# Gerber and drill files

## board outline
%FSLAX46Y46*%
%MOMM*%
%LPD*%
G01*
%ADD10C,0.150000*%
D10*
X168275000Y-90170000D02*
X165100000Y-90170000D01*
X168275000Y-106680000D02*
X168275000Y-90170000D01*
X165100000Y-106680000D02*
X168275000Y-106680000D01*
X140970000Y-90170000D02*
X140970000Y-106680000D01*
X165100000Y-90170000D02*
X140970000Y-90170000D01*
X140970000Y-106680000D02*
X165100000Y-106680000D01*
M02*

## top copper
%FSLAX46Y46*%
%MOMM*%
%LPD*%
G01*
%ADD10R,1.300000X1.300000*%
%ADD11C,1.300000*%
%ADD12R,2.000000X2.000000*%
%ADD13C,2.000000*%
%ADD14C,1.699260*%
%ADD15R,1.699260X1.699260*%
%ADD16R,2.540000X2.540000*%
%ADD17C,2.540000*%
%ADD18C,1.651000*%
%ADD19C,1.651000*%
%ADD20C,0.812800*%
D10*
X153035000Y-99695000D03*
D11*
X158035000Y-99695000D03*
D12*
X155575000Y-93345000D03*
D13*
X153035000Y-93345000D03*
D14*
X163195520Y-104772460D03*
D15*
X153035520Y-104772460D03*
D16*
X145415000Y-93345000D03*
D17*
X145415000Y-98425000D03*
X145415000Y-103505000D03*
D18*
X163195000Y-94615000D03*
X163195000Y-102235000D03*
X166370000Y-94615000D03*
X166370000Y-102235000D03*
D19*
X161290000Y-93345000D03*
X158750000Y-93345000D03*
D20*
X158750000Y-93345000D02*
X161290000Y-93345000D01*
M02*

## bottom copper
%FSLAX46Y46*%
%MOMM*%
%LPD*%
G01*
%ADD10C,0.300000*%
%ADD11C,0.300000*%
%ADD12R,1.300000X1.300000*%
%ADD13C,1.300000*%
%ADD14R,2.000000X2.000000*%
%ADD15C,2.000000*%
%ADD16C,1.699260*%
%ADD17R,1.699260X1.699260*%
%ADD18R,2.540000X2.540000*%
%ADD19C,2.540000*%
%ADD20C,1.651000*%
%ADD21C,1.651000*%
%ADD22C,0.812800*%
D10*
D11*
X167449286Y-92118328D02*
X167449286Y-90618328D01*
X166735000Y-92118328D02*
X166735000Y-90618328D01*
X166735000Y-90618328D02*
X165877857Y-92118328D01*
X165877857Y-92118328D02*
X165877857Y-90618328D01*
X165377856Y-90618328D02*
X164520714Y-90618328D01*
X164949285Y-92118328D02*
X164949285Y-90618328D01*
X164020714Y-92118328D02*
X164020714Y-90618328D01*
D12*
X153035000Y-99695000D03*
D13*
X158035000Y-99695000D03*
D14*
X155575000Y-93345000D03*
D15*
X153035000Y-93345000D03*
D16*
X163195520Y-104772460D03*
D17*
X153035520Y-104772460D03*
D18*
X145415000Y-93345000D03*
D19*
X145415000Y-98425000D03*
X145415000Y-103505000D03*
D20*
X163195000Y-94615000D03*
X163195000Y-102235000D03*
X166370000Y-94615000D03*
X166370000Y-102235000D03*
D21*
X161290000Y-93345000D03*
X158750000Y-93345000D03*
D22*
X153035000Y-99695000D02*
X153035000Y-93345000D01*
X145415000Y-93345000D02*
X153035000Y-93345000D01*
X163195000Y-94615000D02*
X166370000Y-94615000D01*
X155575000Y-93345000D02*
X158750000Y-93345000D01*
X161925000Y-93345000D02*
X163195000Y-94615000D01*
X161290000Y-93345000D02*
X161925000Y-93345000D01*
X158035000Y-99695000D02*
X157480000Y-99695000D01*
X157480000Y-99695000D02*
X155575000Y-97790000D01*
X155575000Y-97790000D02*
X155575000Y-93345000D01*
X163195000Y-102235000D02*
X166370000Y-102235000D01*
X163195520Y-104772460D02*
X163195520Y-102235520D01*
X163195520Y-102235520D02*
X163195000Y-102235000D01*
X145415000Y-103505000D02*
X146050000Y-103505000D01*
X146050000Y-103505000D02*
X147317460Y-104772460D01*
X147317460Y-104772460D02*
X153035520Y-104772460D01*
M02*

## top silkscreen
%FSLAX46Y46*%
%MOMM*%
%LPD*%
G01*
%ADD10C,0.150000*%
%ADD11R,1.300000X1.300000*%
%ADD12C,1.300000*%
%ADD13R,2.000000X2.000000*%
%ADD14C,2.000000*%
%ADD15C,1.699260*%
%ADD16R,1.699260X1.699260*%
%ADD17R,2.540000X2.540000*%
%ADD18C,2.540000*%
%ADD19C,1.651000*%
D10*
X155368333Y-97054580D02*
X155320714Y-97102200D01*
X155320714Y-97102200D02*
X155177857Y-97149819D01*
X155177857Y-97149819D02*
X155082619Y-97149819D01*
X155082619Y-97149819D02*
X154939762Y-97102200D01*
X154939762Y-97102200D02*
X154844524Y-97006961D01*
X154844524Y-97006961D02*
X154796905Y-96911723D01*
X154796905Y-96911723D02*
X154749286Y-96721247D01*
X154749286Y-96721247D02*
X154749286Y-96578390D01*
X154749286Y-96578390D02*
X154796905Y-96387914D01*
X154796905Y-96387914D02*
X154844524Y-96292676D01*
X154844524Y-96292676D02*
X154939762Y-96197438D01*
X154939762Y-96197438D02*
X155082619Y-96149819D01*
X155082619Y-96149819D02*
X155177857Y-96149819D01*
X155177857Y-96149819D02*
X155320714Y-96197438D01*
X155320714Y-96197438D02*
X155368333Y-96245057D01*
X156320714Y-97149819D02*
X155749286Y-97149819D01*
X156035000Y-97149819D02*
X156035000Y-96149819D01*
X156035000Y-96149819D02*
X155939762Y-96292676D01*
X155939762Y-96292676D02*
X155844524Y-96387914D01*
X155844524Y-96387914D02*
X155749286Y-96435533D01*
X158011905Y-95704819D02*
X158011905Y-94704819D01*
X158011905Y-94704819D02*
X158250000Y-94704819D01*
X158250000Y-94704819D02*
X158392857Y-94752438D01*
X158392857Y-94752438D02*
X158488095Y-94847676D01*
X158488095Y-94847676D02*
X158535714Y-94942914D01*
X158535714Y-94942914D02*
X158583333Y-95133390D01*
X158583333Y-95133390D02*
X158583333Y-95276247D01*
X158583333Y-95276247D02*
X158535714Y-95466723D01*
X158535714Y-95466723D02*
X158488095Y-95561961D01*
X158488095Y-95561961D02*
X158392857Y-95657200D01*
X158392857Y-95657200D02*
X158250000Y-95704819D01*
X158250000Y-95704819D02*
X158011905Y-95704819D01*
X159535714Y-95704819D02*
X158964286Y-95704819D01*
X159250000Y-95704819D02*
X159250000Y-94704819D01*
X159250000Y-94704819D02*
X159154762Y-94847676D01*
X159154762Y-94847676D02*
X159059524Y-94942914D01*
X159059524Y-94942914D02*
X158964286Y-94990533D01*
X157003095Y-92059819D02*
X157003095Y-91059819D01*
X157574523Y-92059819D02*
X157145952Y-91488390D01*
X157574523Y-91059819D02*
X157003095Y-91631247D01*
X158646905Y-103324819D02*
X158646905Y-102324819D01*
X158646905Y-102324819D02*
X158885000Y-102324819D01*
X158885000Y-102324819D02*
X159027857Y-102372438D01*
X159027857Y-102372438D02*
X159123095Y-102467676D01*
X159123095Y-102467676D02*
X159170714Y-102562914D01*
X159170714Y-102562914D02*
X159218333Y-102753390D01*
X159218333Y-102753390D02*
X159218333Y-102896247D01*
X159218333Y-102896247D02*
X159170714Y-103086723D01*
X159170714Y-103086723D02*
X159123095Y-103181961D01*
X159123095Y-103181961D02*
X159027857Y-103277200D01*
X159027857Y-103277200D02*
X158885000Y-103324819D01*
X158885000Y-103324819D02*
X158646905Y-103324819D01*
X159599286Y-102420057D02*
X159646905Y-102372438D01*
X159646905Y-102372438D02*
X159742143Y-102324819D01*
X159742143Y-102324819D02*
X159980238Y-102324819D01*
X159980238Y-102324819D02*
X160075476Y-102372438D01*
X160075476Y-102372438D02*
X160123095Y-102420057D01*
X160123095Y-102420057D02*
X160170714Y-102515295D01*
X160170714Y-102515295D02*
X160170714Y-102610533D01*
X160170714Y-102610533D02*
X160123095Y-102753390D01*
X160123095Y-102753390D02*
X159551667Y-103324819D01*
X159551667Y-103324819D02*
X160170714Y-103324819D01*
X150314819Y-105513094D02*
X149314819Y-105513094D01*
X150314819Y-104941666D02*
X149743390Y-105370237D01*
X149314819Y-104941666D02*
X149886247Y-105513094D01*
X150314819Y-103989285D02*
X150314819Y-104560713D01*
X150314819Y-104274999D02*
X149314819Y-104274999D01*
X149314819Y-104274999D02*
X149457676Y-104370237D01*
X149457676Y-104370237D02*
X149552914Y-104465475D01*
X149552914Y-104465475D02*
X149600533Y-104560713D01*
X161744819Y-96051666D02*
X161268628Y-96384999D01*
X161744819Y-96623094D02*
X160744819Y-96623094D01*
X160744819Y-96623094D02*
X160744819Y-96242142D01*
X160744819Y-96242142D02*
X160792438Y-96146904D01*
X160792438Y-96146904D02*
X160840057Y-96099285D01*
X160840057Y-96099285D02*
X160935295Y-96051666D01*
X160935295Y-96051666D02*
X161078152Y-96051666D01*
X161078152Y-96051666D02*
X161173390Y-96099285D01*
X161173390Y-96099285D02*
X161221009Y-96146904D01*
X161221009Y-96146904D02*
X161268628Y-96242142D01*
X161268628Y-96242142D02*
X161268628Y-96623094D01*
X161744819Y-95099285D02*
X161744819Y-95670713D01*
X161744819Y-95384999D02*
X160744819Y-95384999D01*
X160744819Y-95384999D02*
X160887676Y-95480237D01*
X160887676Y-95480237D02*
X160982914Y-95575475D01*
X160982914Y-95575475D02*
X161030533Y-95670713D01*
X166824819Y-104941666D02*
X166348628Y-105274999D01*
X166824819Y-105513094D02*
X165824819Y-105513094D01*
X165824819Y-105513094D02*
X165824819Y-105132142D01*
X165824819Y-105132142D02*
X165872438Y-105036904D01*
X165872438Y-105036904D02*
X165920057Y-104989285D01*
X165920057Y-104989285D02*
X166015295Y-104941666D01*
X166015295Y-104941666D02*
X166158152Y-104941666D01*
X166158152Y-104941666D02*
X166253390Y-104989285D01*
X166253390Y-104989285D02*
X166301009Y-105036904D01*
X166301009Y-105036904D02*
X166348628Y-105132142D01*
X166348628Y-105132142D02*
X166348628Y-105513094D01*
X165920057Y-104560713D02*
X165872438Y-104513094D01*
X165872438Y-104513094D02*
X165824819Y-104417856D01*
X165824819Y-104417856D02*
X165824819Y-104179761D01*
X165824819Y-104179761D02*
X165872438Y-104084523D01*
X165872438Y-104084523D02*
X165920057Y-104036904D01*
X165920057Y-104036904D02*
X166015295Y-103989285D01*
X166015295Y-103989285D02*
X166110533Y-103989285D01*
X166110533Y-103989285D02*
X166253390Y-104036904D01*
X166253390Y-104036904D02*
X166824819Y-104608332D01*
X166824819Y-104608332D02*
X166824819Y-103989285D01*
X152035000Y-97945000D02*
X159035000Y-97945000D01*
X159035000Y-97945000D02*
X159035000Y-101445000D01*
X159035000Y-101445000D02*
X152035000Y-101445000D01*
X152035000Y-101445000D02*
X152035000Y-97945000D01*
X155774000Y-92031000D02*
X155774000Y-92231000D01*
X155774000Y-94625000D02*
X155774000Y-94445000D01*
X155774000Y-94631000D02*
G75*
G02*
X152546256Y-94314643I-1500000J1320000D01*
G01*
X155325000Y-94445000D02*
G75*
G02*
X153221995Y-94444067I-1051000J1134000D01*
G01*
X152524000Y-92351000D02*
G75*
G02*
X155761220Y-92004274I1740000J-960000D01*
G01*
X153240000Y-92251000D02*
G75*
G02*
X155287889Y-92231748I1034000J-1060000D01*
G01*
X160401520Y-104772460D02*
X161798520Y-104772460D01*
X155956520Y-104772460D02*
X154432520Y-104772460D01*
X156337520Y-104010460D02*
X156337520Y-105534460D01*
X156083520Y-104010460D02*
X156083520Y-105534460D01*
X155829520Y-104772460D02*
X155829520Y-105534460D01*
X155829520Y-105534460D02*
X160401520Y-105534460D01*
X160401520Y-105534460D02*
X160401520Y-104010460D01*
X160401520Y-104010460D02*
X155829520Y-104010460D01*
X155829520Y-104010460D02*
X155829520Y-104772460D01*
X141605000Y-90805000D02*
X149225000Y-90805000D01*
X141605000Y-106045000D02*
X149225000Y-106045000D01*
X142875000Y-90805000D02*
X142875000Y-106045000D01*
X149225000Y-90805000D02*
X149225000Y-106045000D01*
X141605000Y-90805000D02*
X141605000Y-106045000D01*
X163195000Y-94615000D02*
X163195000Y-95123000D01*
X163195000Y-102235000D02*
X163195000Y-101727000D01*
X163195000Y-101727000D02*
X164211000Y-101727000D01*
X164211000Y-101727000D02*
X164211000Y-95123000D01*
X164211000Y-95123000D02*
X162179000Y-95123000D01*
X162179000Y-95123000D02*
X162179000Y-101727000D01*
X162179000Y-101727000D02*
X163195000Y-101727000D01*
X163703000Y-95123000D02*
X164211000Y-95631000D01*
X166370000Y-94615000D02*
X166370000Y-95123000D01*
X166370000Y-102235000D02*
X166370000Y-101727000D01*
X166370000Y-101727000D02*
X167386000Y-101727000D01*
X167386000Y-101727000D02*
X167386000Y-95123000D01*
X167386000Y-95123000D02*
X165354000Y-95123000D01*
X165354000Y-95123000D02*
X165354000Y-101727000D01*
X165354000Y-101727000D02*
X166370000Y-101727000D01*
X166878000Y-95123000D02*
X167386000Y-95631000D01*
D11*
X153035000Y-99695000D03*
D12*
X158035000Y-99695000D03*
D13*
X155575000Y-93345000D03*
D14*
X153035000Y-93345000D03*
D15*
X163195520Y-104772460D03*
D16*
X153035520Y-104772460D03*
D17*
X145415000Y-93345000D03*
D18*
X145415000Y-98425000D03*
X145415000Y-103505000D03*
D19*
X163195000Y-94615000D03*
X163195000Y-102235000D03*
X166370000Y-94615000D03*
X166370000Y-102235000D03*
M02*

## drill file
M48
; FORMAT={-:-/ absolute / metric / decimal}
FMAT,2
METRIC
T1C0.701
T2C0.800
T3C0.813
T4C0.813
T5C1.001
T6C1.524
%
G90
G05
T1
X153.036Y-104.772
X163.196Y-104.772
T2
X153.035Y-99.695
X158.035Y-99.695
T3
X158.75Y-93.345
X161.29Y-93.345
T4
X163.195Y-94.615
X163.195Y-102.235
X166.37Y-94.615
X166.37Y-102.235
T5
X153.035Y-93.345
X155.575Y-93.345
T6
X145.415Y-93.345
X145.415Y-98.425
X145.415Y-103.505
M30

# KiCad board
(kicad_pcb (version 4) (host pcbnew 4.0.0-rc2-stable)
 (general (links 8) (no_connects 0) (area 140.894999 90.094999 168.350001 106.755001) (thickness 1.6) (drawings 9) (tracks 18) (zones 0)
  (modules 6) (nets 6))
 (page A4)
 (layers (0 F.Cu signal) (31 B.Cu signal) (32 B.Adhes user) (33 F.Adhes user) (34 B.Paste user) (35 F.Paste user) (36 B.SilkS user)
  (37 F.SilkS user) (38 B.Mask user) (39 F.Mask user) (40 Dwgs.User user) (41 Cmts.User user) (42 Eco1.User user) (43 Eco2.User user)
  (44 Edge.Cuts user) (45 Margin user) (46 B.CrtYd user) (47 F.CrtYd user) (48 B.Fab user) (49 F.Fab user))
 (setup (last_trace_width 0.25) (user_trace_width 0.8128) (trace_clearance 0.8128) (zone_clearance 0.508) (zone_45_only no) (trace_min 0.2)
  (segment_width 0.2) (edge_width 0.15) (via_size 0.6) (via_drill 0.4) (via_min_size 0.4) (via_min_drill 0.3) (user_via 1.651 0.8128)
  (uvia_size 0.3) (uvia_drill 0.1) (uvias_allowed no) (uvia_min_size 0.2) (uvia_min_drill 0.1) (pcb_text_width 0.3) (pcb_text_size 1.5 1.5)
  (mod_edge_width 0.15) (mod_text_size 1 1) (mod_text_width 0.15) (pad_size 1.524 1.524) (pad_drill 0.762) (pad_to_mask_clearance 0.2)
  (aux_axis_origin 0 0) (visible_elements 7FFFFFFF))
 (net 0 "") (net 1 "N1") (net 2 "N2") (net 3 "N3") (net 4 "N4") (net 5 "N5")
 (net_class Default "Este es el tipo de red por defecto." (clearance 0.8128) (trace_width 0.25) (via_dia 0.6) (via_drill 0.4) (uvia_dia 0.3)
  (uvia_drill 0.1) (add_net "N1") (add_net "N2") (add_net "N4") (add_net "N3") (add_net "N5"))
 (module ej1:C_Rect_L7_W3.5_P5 (layer F.Cu) (at 153.035 99.695)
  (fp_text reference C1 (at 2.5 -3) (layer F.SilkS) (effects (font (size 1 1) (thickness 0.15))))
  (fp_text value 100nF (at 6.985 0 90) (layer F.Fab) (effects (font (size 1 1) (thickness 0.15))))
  (fp_line (start -1 -1.75) (end 6 -1.75) (layer F.SilkS) (width 0.15))
  (fp_line (start 6 -1.75) (end 6 1.75) (layer F.SilkS) (width 0.15))
  (fp_line (start 6 1.75) (end -1 1.75) (layer F.SilkS) (width 0.15))
  (fp_line (start -1 1.75) (end -1 -1.75) (layer F.SilkS) (width 0.15))
  (pad 1 thru_hole rect (at 0 0) (size 1.3 1.3) (drill 0.8) (layers *.Cu *.Mask F.SilkS) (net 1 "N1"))
  (pad 2 thru_hole circle (at 5 0) (size 1.3 1.3) (drill 0.8) (layers *.Cu *.Mask F.SilkS) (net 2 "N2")))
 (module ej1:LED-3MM (layer F.Cu) (at 155.575 93.345 180)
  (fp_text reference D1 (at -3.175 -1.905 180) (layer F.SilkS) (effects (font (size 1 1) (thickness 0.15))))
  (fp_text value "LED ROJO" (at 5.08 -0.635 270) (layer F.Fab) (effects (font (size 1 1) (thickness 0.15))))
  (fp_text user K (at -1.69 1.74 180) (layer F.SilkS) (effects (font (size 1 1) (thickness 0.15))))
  (fp_line (start -0.199 1.314) (end -0.199 1.114) (layer F.SilkS) (width 0.15))
  (fp_line (start -0.199 -1.28) (end -0.199 -1.1) (layer F.SilkS) (width 0.15))
  (fp_arc (start 1.301 0.034) (end -0.199 -1.286) (angle 108.5) (layer F.SilkS) (width 0.15))
  (fp_arc (start 1.301 0.034) (end 0.25 -1.1) (angle 85.7) (layer F.SilkS) (width 0.15))
  (fp_arc (start 1.311 0.034) (end 3.051 0.994) (angle 110) (layer F.SilkS) (width 0.15))
  (fp_arc (start 1.301 0.034) (end 2.335 1.094) (angle 87.5) (layer F.SilkS) (width 0.15))
  (pad 1 thru_hole rect (at 0 0 270) (size 2 2) (drill 1.00076) (layers *.Cu *.Mask F.SilkS) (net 2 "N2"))
  (pad 2 thru_hole circle (at 2.54 0 180) (size 2 2) (drill 1.00076) (layers *.Cu *.Mask F.SilkS) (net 1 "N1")))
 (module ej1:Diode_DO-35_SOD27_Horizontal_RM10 (layer F.Cu) (at 153.035 104.775)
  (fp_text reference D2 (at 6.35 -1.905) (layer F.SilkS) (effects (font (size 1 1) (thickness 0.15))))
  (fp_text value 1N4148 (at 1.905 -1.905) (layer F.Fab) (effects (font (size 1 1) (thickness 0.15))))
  (fp_line (start 7.36652 -0.00254) (end 8.76352 -0.00254) (layer F.SilkS) (width 0.15))
  (fp_line (start 2.92152 -0.00254) (end 1.39752 -0.00254) (layer F.SilkS) (width 0.15))
  (fp_line (start 3.30252 -0.76454) (end 3.30252 0.75946) (layer F.SilkS) (width 0.15))
  (fp_line (start 3.04852 -0.76454) (end 3.04852 0.75946) (layer F.SilkS) (width 0.15))
  (fp_line (start 2.79452 -0.00254) (end 2.79452 0.75946) (layer F.SilkS) (width 0.15))
  (fp_line (start 2.79452 0.75946) (end 7.36652 0.75946) (layer F.SilkS) (width 0.15))
  (fp_line (start 7.36652 0.75946) (end 7.36652 -0.76454) (layer F.SilkS) (width 0.15))
  (fp_line (start 7.36652 -0.76454) (end 2.79452 -0.76454) (layer F.SilkS) (width 0.15))
  (fp_line (start 2.79452 -0.76454) (end 2.79452 -0.00254) (layer F.SilkS) (width 0.15))
  (pad 2 thru_hole circle (at 10.16052 -0.00254 180) (size 1.69926 1.69926) (drill 0.70104) (layers *.Cu *.Mask F.SilkS) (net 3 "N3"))
  (pad 1 thru_hole rect (at 0.00052 -0.00254 180) (size 1.69926 1.69926) (drill 0.70104) (layers *.Cu *.Mask F.SilkS) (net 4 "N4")))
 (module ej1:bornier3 (layer F.Cu) (at 145.415 98.425 270)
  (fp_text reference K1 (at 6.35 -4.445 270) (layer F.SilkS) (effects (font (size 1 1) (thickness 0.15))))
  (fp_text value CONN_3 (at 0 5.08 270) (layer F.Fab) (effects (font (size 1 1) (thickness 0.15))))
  (fp_line (start -7.62 3.81) (end -7.62 -3.81) (layer F.SilkS) (width 0.15))
  (fp_line (start 7.62 3.81) (end 7.62 -3.81) (layer F.SilkS) (width 0.15))
  (fp_line (start -7.62 2.54) (end 7.62 2.54) (layer F.SilkS) (width 0.15))
  (fp_line (start -7.62 -3.81) (end 7.62 -3.81) (layer F.SilkS) (width 0.15))
  (fp_line (start -7.62 3.81) (end 7.62 3.81) (layer F.SilkS) (width 0.15))
  (pad 1 thru_hole rect (at -5.08 0 270) (size 2.54 2.54) (drill 1.524) (layers *.Cu *.Mask F.SilkS) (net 1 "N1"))
  (pad 2 thru_hole circle (at 0 0 270) (size 2.54 2.54) (drill 1.524) (layers *.Cu *.Mask F.SilkS) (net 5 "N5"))
  (pad 3 thru_hole circle (at 5.08 0 270) (size 2.54 2.54) (drill 1.524) (layers *.Cu *.Mask F.SilkS) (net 4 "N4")))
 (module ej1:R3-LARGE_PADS (layer F.Cu) (at 163.195 98.425 270)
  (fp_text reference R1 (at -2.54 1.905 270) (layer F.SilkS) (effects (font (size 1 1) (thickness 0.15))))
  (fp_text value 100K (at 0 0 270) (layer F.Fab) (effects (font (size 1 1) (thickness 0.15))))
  (fp_line (start -3.81 0) (end -3.302 0) (layer F.SilkS) (width 0.15))
  (fp_line (start 3.81 0) (end 3.302 0) (layer F.SilkS) (width 0.15))
  (fp_line (start 3.302 0) (end 3.302 -1.016) (layer F.SilkS) (width 0.15))
  (fp_line (start 3.302 -1.016) (end -3.302 -1.016) (layer F.SilkS) (width 0.15))
  (fp_line (start -3.302 -1.016) (end -3.302 1.016) (layer F.SilkS) (width 0.15))
  (fp_line (start -3.302 1.016) (end 3.302 1.016) (layer F.SilkS) (width 0.15))
  (fp_line (start 3.302 1.016) (end 3.302 0) (layer F.SilkS) (width 0.15))
  (fp_line (start -3.302 -0.508) (end -2.794 -1.016) (layer F.SilkS) (width 0.15))
  (pad 1 thru_hole circle (at -3.81 0 270) (size 1.651 1.651) (drill 0.8128) (layers *.Cu *.Mask F.SilkS) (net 2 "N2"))
  (pad 2 thru_hole circle (at 3.81 0 270) (size 1.651 1.651) (drill 0.8128) (layers *.Cu *.Mask F.SilkS) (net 3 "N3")))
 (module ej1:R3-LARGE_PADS (layer F.Cu) (at 166.37 98.425 270)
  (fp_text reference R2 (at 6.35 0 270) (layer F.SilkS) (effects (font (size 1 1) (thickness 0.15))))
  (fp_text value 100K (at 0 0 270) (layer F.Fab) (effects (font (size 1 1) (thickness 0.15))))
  (fp_line (start -3.81 0) (end -3.302 0) (layer F.SilkS) (width 0.15))
  (fp_line (start 3.81 0) (end 3.302 0) (layer F.SilkS) (width 0.15))
  (fp_line (start 3.302 0) (end 3.302 -1.016) (layer F.SilkS) (width 0.15))
  (fp_line (start 3.302 -1.016) (end -3.302 -1.016) (layer F.SilkS) (width 0.15))
  (fp_line (start -3.302 -1.016) (end -3.302 1.016) (layer F.SilkS) (width 0.15))
  (fp_line (start -3.302 1.016) (end 3.302 1.016) (layer F.SilkS) (width 0.15))
  (fp_line (start 3.302 1.016) (end 3.302 0) (layer F.SilkS) (width 0.15))
  (fp_line (start -3.302 -0.508) (end -2.794 -1.016) (layer F.SilkS) (width 0.15))
  (pad 1 thru_hole circle (at -3.81 0 270) (size 1.651 1.651) (drill 0.8128) (layers *.Cu *.Mask F.SilkS) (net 2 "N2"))
  (pad 2 thru_hole circle (at 3.81 0 270) (size 1.651 1.651) (drill 0.8128) (layers *.Cu *.Mask F.SilkS) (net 3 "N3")))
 (gr_line (start 168.275 90.17) (end 165.1 90.17) (angle 90) (layer Edge.Cuts) (width 0.15))
 (gr_line (start 168.275 106.68) (end 168.275 90.17) (angle 90) (layer Edge.Cuts) (width 0.15))
 (gr_line (start 165.1 106.68) (end 168.275 106.68) (angle 90) (layer Edge.Cuts) (width 0.15))
 (gr_line (start 140.97 90.17) (end 140.97 106.68) (angle 90) (layer Edge.Cuts) (width 0.15))
 (gr_line (start 165.1 90.17) (end 140.97 90.17) (angle 90) (layer Edge.Cuts) (width 0.15))
 (gr_line (start 140.97 106.68) (end 165.1 106.68) (angle 90) (layer Edge.Cuts) (width 0.15))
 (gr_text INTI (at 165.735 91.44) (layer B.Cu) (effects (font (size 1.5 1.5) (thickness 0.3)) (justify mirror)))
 (segment (start 153.035 99.695) (end 153.035 93.345) (width 0.8128) (layer B.Cu) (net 1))
 (segment (start 145.415 93.345) (end 153.035 93.345) (width 0.8128) (layer B.Cu) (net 1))
 (segment (start 163.195 94.615) (end 166.37 94.615) (width 0.8128) (layer B.Cu) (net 2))
 (segment (start 155.575 93.345) (end 158.75 93.345) (width 0.8128) (layer B.Cu) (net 2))
 (segment (start 161.925 93.345) (end 163.195 94.615) (width 0.8128) (layer B.Cu) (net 2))
 (segment (start 161.29 93.345) (end 161.925 93.345) (width 0.8128) (layer B.Cu) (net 2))
 (segment (start 158.75 93.345) (end 161.29 93.345) (width 0.8128) (layer F.Cu) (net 2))
 (segment (start 158.035 99.695) (end 157.48 99.695) (width 0.8128) (layer B.Cu) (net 2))
 (segment (start 157.48 99.695) (end 155.575 97.79) (width 0.8128) (layer B.Cu) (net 2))
 (segment (start 155.575 97.79) (end 155.575 93.345) (width 0.8128) (layer B.Cu) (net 2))
 (segment (start 163.195 102.235) (end 166.37 102.235) (width 0.8128) (layer B.Cu) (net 3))
 (segment (start 163.19552 104.77246) (end 163.19552 102.23552) (width 0.8128) (layer B.Cu) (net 3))
 (segment (start 163.19552 102.23552) (end 163.195 102.235) (width 0.8128) (layer B.Cu) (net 3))
 (segment (start 145.415 103.505) (end 146.05 103.505) (width 0.8128) (layer B.Cu) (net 4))
 (segment (start 146.05 103.505) (end 147.31746 104.77246) (width 0.8128) (layer B.Cu) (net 4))
 (segment (start 147.31746 104.77246) (end 153.03552 104.77246) (width 0.8128) (layer B.Cu) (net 4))
 (via (at 161.29 93.345) (size 1.651) (drill 0.8128) (layers F.Cu B.Cu) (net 2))
 (via (at 158.75 93.345) (size 1.651) (drill 0.8128) (layers F.Cu B.Cu) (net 2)))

